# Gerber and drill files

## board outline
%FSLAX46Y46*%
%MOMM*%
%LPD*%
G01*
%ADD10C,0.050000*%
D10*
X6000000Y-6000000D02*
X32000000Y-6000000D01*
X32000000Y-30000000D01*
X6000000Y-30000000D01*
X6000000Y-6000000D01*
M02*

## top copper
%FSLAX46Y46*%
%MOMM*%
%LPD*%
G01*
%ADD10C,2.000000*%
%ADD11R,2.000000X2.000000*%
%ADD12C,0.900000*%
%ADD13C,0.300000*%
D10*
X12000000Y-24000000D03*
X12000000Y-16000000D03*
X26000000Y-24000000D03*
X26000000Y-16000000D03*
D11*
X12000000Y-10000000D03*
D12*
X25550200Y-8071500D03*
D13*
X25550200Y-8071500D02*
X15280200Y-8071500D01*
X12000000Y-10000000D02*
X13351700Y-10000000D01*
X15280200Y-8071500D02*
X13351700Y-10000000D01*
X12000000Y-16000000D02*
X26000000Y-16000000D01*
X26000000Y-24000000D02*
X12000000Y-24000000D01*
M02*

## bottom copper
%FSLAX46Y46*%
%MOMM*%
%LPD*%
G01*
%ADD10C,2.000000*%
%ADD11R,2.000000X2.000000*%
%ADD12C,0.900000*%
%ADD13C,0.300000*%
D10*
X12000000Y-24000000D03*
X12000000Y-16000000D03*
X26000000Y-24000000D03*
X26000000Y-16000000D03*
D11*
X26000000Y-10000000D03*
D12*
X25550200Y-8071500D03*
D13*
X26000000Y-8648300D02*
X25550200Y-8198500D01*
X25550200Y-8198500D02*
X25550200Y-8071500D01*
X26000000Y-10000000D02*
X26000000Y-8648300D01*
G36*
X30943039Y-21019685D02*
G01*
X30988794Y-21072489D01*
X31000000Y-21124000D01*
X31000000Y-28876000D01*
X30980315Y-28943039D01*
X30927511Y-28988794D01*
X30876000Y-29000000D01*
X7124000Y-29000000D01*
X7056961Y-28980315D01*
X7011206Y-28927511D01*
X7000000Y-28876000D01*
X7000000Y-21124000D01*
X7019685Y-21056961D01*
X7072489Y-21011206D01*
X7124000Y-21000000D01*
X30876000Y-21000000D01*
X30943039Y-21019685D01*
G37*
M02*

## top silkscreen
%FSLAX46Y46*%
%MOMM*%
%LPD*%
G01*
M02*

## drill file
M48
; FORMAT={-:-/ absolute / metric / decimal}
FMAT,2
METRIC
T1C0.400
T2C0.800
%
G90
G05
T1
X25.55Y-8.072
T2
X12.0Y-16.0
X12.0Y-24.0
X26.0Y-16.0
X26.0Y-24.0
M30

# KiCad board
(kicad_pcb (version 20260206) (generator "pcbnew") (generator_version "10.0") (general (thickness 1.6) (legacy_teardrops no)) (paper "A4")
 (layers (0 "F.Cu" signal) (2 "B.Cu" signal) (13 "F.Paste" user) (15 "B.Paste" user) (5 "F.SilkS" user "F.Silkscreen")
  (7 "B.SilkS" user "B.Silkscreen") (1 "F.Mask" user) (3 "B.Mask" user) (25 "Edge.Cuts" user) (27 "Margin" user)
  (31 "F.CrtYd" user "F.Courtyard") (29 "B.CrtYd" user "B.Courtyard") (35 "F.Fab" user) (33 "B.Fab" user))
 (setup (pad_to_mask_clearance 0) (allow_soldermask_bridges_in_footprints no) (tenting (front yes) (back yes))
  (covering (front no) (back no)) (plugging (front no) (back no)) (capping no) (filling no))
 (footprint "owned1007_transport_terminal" (layer "F.Cu") (at 12 24)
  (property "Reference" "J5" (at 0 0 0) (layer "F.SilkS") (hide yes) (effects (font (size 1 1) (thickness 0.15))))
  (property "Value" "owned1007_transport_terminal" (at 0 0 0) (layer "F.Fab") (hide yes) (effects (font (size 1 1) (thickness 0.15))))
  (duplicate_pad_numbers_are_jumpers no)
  (pad "1" thru_hole circle (at 0 0) (size 2 2) (drill 0.8) (layers "*.Cu" "*.Mask") (remove_unused_layers no) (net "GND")))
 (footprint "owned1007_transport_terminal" (layer "F.Cu") (at 12 16)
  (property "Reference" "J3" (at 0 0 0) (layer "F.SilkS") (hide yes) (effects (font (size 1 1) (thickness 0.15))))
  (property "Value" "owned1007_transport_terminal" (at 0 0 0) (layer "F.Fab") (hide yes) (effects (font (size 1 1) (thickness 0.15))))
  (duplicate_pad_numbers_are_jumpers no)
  (pad "1" thru_hole circle (at 0 0) (size 2 2) (drill 0.8) (layers "*.Cu" "*.Mask") (remove_unused_layers no) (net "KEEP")))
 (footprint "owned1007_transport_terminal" (layer "F.Cu") (at 26 24)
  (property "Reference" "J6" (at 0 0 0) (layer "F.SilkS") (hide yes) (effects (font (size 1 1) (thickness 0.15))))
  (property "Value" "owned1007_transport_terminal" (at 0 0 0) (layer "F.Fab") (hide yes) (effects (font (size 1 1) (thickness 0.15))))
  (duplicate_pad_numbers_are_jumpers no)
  (pad "1" thru_hole circle (at 0 0) (size 2 2) (drill 0.8) (layers "*.Cu" "*.Mask") (remove_unused_layers no) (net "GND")))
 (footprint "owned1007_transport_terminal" (layer "F.Cu") (at 26 16)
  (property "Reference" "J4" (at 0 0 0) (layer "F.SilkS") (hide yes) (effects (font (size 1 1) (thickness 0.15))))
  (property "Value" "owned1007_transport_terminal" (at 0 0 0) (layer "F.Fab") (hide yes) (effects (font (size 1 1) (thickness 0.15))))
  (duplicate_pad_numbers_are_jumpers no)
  (pad "1" thru_hole circle (at 0 0) (size 2 2) (drill 0.8) (layers "*.Cu" "*.Mask") (remove_unused_layers no) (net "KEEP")))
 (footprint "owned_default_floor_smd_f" (layer "F.Cu") (at 12 10)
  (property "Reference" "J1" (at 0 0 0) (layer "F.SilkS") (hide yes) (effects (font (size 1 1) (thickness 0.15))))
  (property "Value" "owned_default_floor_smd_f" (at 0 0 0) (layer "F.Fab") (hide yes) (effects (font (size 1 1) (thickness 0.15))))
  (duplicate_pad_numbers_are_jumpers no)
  (pad "1" smd rect (at 0 0) (size 2 2) (layers "F.Cu" "F.Mask" "F.Paste") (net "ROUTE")))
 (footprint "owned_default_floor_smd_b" (layer "B.Cu") (at 26 10)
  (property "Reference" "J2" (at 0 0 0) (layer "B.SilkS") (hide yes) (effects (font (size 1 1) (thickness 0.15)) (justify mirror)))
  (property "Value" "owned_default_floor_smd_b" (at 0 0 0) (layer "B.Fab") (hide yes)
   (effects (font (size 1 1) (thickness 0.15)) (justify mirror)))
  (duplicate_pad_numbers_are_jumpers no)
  (pad "1" smd rect (at 0 0) (size 2 2) (layers "B.Cu" "B.Mask" "B.Paste") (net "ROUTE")))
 (gr_rect (start 6 6) (end 32 30) (stroke (width 0.05) (type default)) (fill no) (layer "Edge.Cuts"))
 (segment (start 25.5502 8.0715) (end 15.2802 8.0715) (width 0.3) (layer "F.Cu") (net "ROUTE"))
 (segment (start 12 10) (end 13.3517 10) (width 0.3) (layer "F.Cu") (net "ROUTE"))
 (segment (start 15.2802 8.0715) (end 13.3517 10) (width 0.3) (layer "F.Cu") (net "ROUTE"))
 (via (at 25.5502 8.0715) (size 0.9) (drill 0.4) (layers "F.Cu" "B.Cu") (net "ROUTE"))
 (segment (start 26 8.6483) (end 25.5502 8.1985) (width 0.3) (layer "B.Cu") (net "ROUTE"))
 (segment (start 25.5502 8.1985) (end 25.5502 8.0715) (width 0.3) (layer "B.Cu") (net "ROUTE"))
 (segment (start 26 10) (end 26 8.6483) (width 0.3) (layer "B.Cu") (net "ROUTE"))
 (segment (start 12 16) (end 26 16) (width 0.3) (locked yes) (layer "F.Cu") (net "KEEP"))
 (segment (start 26 24) (end 12 24) (width 0.3) (layer "F.Cu") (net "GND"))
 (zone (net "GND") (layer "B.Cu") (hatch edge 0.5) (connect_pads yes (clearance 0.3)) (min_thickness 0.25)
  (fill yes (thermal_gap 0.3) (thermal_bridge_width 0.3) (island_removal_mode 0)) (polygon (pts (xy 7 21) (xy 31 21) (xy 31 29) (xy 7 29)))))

